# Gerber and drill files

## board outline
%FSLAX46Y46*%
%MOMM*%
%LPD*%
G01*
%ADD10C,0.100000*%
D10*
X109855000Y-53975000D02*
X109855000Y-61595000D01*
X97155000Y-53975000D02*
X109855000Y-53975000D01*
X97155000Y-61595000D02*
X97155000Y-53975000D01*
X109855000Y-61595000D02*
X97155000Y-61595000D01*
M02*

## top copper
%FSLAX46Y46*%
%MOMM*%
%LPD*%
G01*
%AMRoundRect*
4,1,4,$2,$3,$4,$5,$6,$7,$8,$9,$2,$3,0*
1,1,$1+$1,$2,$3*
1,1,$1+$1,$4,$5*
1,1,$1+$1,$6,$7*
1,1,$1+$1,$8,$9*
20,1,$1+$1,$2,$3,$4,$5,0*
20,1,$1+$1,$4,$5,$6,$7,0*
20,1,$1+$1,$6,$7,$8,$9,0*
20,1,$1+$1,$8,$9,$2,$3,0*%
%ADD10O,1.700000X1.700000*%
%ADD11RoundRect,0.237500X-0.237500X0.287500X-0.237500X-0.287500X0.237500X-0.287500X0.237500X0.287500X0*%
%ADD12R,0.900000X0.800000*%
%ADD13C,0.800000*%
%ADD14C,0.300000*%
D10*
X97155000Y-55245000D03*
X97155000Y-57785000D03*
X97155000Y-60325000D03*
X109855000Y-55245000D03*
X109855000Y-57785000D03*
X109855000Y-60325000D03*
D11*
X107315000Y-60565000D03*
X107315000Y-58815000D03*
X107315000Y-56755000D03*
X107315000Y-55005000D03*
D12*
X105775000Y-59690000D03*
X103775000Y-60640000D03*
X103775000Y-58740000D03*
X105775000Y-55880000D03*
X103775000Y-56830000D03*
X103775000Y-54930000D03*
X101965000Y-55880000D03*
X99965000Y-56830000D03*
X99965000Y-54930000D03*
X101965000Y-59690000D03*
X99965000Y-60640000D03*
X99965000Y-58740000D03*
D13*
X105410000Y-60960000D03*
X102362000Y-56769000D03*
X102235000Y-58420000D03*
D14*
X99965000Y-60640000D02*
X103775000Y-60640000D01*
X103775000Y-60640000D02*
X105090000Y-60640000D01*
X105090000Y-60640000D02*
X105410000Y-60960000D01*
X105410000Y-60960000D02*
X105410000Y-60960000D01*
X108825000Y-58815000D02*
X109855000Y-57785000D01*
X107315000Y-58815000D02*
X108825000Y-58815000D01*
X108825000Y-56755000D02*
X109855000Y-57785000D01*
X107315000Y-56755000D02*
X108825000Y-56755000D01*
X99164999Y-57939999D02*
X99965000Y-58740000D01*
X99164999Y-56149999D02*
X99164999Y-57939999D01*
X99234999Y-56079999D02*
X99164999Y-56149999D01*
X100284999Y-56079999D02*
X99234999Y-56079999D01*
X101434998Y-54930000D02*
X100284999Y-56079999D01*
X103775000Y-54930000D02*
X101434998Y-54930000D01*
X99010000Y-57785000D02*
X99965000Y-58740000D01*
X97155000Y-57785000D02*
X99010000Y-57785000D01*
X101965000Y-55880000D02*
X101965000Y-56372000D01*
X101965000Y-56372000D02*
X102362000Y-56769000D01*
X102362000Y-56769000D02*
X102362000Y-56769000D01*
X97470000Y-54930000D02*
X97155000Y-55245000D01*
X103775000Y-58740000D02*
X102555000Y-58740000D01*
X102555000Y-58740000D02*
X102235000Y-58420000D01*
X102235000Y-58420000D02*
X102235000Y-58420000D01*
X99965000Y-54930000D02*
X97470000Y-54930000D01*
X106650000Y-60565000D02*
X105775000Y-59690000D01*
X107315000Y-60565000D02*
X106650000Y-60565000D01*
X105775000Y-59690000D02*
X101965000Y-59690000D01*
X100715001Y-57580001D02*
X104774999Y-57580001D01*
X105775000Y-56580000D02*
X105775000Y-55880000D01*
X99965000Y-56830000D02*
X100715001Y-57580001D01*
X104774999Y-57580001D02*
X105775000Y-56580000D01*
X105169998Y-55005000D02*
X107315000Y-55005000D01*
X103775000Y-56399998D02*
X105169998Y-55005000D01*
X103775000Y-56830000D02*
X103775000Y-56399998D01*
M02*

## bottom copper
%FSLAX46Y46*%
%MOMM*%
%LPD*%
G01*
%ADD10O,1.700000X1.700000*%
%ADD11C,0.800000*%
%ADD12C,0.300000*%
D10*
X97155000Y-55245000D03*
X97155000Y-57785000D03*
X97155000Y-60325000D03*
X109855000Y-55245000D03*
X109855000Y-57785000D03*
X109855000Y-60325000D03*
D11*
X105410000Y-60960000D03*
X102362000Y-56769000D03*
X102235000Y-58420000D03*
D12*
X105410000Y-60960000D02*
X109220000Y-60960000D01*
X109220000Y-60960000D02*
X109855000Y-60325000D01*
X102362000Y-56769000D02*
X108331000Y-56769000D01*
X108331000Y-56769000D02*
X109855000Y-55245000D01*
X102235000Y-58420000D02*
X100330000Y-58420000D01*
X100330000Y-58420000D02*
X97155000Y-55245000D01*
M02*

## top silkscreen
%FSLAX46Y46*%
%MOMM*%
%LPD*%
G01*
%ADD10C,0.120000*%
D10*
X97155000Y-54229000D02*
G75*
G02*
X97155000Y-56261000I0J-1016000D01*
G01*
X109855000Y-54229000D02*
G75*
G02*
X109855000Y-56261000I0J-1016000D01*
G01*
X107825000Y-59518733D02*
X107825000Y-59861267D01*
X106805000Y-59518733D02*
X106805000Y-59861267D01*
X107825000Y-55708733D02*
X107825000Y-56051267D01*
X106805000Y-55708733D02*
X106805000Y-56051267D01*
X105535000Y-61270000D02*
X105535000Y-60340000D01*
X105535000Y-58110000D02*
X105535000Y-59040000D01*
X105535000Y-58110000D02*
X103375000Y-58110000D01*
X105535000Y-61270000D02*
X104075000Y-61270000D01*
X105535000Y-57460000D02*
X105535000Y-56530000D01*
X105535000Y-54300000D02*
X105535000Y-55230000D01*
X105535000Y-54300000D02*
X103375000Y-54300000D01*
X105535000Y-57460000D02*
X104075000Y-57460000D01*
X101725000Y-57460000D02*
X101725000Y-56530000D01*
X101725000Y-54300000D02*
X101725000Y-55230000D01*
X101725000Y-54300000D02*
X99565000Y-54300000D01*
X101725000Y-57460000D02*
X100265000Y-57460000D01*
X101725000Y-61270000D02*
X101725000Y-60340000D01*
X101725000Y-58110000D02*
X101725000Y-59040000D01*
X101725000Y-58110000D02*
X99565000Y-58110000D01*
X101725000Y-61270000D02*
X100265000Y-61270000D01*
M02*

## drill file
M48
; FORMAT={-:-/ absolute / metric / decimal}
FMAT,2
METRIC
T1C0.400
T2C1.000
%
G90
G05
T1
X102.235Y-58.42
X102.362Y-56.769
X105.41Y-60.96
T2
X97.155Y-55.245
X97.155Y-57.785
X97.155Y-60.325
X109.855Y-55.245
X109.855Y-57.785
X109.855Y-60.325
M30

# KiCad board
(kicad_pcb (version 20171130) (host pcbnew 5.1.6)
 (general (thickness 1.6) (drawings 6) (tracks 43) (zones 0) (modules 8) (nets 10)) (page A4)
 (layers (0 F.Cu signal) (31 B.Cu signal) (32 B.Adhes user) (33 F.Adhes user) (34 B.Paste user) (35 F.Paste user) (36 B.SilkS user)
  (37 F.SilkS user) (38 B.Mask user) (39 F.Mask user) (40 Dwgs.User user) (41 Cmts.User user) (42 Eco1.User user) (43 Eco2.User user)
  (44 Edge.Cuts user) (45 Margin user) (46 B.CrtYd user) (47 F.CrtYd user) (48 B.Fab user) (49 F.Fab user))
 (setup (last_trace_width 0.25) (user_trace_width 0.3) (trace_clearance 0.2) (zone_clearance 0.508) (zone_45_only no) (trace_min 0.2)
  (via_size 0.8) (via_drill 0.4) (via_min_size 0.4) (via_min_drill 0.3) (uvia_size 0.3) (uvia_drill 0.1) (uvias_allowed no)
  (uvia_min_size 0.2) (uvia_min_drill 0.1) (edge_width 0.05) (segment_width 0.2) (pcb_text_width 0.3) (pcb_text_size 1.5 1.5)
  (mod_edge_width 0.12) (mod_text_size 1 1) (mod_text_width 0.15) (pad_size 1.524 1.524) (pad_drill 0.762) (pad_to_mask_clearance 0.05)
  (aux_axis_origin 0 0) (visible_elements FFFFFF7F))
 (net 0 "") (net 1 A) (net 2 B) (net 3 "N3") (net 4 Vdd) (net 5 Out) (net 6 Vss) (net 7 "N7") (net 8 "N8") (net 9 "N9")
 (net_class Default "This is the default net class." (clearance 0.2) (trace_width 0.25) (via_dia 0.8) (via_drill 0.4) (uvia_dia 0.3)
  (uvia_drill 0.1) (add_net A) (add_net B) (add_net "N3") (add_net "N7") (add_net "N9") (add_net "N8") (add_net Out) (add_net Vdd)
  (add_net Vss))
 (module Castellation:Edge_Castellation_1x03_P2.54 (layer F.Cu) (at 97.155 55.245)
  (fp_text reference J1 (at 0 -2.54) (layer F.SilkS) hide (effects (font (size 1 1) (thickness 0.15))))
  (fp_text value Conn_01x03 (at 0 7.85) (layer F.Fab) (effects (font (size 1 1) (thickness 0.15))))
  (fp_arc (start 0 0) (end 0 1.016) (angle -180) (layer F.SilkS) (width 0.12))
  (pad 1 thru_hole oval (at 0 0) (size 1.7 1.7) (drill 1) (layers *.Cu *.Mask) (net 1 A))
  (pad 2 thru_hole oval (at 0 2.54) (size 1.7 1.7) (drill 1) (layers *.Cu *.Mask) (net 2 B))
  (pad 3 thru_hole oval (at 0 5.08) (size 1.7 1.7) (drill 1) (layers *.Cu *.Mask) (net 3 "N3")))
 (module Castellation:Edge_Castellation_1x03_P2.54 (layer F.Cu) (at 109.855 55.245)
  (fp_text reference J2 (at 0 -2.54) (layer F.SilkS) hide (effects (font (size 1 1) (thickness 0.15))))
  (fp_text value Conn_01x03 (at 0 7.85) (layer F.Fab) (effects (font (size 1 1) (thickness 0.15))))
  (fp_arc (start 0 0) (end 0 1.016) (angle -180) (layer F.SilkS) (width 0.12))
  (pad 1 thru_hole oval (at 0 0) (size 1.7 1.7) (drill 1) (layers *.Cu *.Mask) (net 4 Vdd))
  (pad 2 thru_hole oval (at 0 2.54) (size 1.7 1.7) (drill 1) (layers *.Cu *.Mask) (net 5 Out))
  (pad 3 thru_hole oval (at 0 5.08) (size 1.7 1.7) (drill 1) (layers *.Cu *.Mask) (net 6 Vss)))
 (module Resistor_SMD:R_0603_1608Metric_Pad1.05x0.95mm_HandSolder (layer F.Cu) (at 107.315 59.69 270)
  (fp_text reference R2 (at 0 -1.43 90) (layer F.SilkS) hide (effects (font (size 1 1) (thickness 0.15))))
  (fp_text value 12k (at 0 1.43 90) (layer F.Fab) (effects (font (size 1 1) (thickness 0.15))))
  (fp_line (start -0.171267 -0.51) (end 0.171267 -0.51) (layer F.SilkS) (width 0.12))
  (fp_line (start -0.171267 0.51) (end 0.171267 0.51) (layer F.SilkS) (width 0.12))
  (pad 2 smd roundrect (at 0.875 0 270) (size 1.05 0.95) (layers F.Cu F.Paste F.Mask) (roundrect_rratio 0.25) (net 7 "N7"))
  (pad 1 smd roundrect (at -0.875 0 270) (size 1.05 0.95) (layers F.Cu F.Paste F.Mask) (roundrect_rratio 0.25) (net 5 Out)))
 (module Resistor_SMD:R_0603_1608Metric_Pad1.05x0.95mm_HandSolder (layer F.Cu) (at 107.315 55.88 270)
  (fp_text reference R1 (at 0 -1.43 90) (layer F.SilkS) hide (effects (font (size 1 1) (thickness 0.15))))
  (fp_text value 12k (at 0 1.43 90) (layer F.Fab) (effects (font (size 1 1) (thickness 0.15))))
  (fp_line (start -0.171267 -0.51) (end 0.171267 -0.51) (layer F.SilkS) (width 0.12))
  (fp_line (start -0.171267 0.51) (end 0.171267 0.51) (layer F.SilkS) (width 0.12))
  (pad 2 smd roundrect (at 0.875 0 270) (size 1.05 0.95) (layers F.Cu F.Paste F.Mask) (roundrect_rratio 0.25) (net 5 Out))
  (pad 1 smd roundrect (at -0.875 0 270) (size 1.05 0.95) (layers F.Cu F.Paste F.Mask) (roundrect_rratio 0.25) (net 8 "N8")))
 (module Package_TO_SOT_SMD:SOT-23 (layer F.Cu) (at 104.775 59.69)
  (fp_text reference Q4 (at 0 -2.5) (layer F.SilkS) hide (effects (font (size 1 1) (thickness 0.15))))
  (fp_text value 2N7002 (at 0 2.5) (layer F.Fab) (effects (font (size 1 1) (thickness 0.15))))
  (fp_line (start 0.76 1.58) (end 0.76 0.65) (layer F.SilkS) (width 0.12))
  (fp_line (start 0.76 -1.58) (end 0.76 -0.65) (layer F.SilkS) (width 0.12))
  (fp_line (start 0.76 -1.58) (end -1.4 -1.58) (layer F.SilkS) (width 0.12))
  (fp_line (start 0.76 1.58) (end -0.7 1.58) (layer F.SilkS) (width 0.12))
  (pad 3 smd rect (at 1 0) (size 0.9 0.8) (layers F.Cu F.Paste F.Mask) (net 7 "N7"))
  (pad 2 smd rect (at -1 0.95) (size 0.9 0.8) (layers F.Cu F.Paste F.Mask) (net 6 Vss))
  (pad 1 smd rect (at -1 -0.95) (size 0.9 0.8) (layers F.Cu F.Paste F.Mask) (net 1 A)))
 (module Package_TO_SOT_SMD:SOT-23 (layer F.Cu) (at 104.775 55.88)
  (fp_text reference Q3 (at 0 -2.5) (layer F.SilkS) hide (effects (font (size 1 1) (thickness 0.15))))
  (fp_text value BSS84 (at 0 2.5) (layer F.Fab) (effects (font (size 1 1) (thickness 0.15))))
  (fp_line (start 0.76 1.58) (end 0.76 0.65) (layer F.SilkS) (width 0.12))
  (fp_line (start 0.76 -1.58) (end 0.76 -0.65) (layer F.SilkS) (width 0.12))
  (fp_line (start 0.76 -1.58) (end -1.4 -1.58) (layer F.SilkS) (width 0.12))
  (fp_line (start 0.76 1.58) (end -0.7 1.58) (layer F.SilkS) (width 0.12))
  (pad 3 smd rect (at 1 0) (size 0.9 0.8) (layers F.Cu F.Paste F.Mask) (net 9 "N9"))
  (pad 2 smd rect (at -1 0.95) (size 0.9 0.8) (layers F.Cu F.Paste F.Mask) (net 8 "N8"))
  (pad 1 smd rect (at -1 -0.95) (size 0.9 0.8) (layers F.Cu F.Paste F.Mask) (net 2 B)))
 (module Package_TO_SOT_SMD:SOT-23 (layer F.Cu) (at 100.965 55.88)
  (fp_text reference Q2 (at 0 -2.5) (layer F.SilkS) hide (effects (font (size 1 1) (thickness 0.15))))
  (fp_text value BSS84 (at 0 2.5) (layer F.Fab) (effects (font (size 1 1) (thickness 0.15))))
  (fp_line (start 0.76 1.58) (end 0.76 0.65) (layer F.SilkS) (width 0.12))
  (fp_line (start 0.76 -1.58) (end 0.76 -0.65) (layer F.SilkS) (width 0.12))
  (fp_line (start 0.76 -1.58) (end -1.4 -1.58) (layer F.SilkS) (width 0.12))
  (fp_line (start 0.76 1.58) (end -0.7 1.58) (layer F.SilkS) (width 0.12))
  (pad 3 smd rect (at 1 0) (size 0.9 0.8) (layers F.Cu F.Paste F.Mask) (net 4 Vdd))
  (pad 2 smd rect (at -1 0.95) (size 0.9 0.8) (layers F.Cu F.Paste F.Mask) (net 9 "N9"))
  (pad 1 smd rect (at -1 -0.95) (size 0.9 0.8) (layers F.Cu F.Paste F.Mask) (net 1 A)))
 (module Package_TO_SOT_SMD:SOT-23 (layer F.Cu) (at 100.965 59.69)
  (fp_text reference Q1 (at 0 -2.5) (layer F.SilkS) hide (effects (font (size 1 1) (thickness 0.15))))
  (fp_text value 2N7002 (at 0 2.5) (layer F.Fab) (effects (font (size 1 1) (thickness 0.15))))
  (fp_line (start 0.76 1.58) (end 0.76 0.65) (layer F.SilkS) (width 0.12))
  (fp_line (start 0.76 -1.58) (end 0.76 -0.65) (layer F.SilkS) (width 0.12))
  (fp_line (start 0.76 -1.58) (end -1.4 -1.58) (layer F.SilkS) (width 0.12))
  (fp_line (start 0.76 1.58) (end -0.7 1.58) (layer F.SilkS) (width 0.12))
  (pad 3 smd rect (at 1 0) (size 0.9 0.8) (layers F.Cu F.Paste F.Mask) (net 7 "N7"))
  (pad 2 smd rect (at -1 0.95) (size 0.9 0.8) (layers F.Cu F.Paste F.Mask) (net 6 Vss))
  (pad 1 smd rect (at -1 -0.95) (size 0.9 0.8) (layers F.Cu F.Paste F.Mask) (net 2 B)))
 (gr_line (start 109.855 53.975) (end 109.855 61.595) (layer Edge.Cuts) (width 0.1))
 (gr_line (start 97.155 53.975) (end 109.855 53.975) (layer Edge.Cuts) (width 0.1))
 (gr_line (start 97.155 61.595) (end 97.155 53.975) (layer Edge.Cuts) (width 0.1))
 (gr_line (start 109.855 61.595) (end 97.155 61.595) (layer Edge.Cuts) (width 0.1))
 (segment (start 99.965 60.64) (end 103.775 60.64) (width 0.3) (layer F.Cu) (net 6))
 (segment (start 103.775 60.64) (end 105.09 60.64) (width 0.3) (layer F.Cu) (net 6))
 (segment (start 105.09 60.64) (end 105.41 60.96) (width 0.3) (layer F.Cu) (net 6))
 (segment (start 105.41 60.96) (end 105.41 60.96) (width 0.3) (layer F.Cu) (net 6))
 (via (at 105.41 60.96) (size 0.8) (drill 0.4) (layers F.Cu B.Cu) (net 6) (status 1000000))
 (segment (start 105.41 60.96) (end 109.22 60.96) (width 0.3) (layer B.Cu) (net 6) (status 1000000))
 (segment (start 109.22 60.96) (end 109.855 60.325) (width 0.3) (layer B.Cu) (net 6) (status 1000000))
 (segment (start 108.825 58.815) (end 109.855 57.785) (width 0.3) (layer F.Cu) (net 5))
 (segment (start 107.315 58.815) (end 108.825 58.815) (width 0.3) (layer F.Cu) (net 5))
 (segment (start 108.825 56.755) (end 109.855 57.785) (width 0.3) (layer F.Cu) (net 5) (status 1000000))
 (segment (start 107.315 56.755) (end 108.825 56.755) (width 0.3) (layer F.Cu) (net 5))
 (segment (start 99.164999 57.939999) (end 99.965 58.74) (width 0.3) (layer F.Cu) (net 2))
 (segment (start 99.164999 56.149999) (end 99.164999 57.939999) (width 0.3) (layer F.Cu) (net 2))
 (segment (start 99.234999 56.079999) (end 99.164999 56.149999) (width 0.3) (layer F.Cu) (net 2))
 (segment (start 100.284999 56.079999) (end 99.234999 56.079999) (width 0.3) (layer F.Cu) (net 2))
 (segment (start 101.434998 54.93) (end 100.284999 56.079999) (width 0.3) (layer F.Cu) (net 2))
 (segment (start 103.775 54.93) (end 101.434998 54.93) (width 0.3) (layer F.Cu) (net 2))
 (segment (start 99.01 57.785) (end 99.965 58.74) (width 0.3) (layer F.Cu) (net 2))
 (segment (start 97.155 57.785) (end 99.01 57.785) (width 0.3) (layer F.Cu) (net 2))
 (segment (start 101.965 55.88) (end 101.965 56.372) (width 0.3) (layer F.Cu) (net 4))
 (segment (start 101.965 56.372) (end 102.362 56.769) (width 0.3) (layer F.Cu) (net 4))
 (segment (start 102.362 56.769) (end 102.362 56.769) (width 0.3) (layer F.Cu) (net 4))
 (via (at 102.362 56.769) (size 0.8) (drill 0.4) (layers F.Cu B.Cu) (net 4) (status 1000000))
 (segment (start 102.362 56.769) (end 108.331 56.769) (width 0.3) (layer B.Cu) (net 4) (status 1000000))
 (segment (start 108.331 56.769) (end 109.855 55.245) (width 0.3) (layer B.Cu) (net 4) (status 1000000))
 (segment (start 97.47 54.93) (end 97.155 55.245) (width 0.3) (layer F.Cu) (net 1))
 (segment (start 103.775 58.74) (end 102.555 58.74) (width 0.3) (layer F.Cu) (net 1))
 (segment (start 102.555 58.74) (end 102.235 58.42) (width 0.3) (layer F.Cu) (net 1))
 (segment (start 102.235 58.42) (end 102.235 58.42) (width 0.3) (layer F.Cu) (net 1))
 (segment (start 99.965 54.93) (end 97.47 54.93) (width 0.3) (layer F.Cu) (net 1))
 (segment (start 102.235 58.42) (end 100.33 58.42) (width 0.3) (layer B.Cu) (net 1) (status 1000000))
 (via (at 102.235 58.42) (size 0.8) (drill 0.4) (layers F.Cu B.Cu) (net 1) (status 1000000))
 (segment (start 100.33 58.42) (end 97.155 55.245) (width 0.3) (layer B.Cu) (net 1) (status 1000000))
 (segment (start 106.65 60.565) (end 105.775 59.69) (width 0.3) (layer F.Cu) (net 7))
 (segment (start 107.315 60.565) (end 106.65 60.565) (width 0.3) (layer F.Cu) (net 7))
 (segment (start 105.775 59.69) (end 101.965 59.69) (width 0.3) (layer F.Cu) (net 7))
 (segment (start 100.715001 57.580001) (end 104.774999 57.580001) (width 0.3) (layer F.Cu) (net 9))
 (segment (start 105.775 56.58) (end 105.775 55.88) (width 0.3) (layer F.Cu) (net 9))
 (segment (start 99.965 56.83) (end 100.715001 57.580001) (width 0.3) (layer F.Cu) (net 9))
 (segment (start 104.774999 57.580001) (end 105.775 56.58) (width 0.3) (layer F.Cu) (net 9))
 (segment (start 105.169998 55.005) (end 107.315 55.005) (width 0.3) (layer F.Cu) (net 8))
 (segment (start 103.775 56.399998) (end 105.169998 55.005) (width 0.3) (layer F.Cu) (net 8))
 (segment (start 103.775 56.83) (end 103.775 56.399998) (width 0.3) (layer F.Cu) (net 8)))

